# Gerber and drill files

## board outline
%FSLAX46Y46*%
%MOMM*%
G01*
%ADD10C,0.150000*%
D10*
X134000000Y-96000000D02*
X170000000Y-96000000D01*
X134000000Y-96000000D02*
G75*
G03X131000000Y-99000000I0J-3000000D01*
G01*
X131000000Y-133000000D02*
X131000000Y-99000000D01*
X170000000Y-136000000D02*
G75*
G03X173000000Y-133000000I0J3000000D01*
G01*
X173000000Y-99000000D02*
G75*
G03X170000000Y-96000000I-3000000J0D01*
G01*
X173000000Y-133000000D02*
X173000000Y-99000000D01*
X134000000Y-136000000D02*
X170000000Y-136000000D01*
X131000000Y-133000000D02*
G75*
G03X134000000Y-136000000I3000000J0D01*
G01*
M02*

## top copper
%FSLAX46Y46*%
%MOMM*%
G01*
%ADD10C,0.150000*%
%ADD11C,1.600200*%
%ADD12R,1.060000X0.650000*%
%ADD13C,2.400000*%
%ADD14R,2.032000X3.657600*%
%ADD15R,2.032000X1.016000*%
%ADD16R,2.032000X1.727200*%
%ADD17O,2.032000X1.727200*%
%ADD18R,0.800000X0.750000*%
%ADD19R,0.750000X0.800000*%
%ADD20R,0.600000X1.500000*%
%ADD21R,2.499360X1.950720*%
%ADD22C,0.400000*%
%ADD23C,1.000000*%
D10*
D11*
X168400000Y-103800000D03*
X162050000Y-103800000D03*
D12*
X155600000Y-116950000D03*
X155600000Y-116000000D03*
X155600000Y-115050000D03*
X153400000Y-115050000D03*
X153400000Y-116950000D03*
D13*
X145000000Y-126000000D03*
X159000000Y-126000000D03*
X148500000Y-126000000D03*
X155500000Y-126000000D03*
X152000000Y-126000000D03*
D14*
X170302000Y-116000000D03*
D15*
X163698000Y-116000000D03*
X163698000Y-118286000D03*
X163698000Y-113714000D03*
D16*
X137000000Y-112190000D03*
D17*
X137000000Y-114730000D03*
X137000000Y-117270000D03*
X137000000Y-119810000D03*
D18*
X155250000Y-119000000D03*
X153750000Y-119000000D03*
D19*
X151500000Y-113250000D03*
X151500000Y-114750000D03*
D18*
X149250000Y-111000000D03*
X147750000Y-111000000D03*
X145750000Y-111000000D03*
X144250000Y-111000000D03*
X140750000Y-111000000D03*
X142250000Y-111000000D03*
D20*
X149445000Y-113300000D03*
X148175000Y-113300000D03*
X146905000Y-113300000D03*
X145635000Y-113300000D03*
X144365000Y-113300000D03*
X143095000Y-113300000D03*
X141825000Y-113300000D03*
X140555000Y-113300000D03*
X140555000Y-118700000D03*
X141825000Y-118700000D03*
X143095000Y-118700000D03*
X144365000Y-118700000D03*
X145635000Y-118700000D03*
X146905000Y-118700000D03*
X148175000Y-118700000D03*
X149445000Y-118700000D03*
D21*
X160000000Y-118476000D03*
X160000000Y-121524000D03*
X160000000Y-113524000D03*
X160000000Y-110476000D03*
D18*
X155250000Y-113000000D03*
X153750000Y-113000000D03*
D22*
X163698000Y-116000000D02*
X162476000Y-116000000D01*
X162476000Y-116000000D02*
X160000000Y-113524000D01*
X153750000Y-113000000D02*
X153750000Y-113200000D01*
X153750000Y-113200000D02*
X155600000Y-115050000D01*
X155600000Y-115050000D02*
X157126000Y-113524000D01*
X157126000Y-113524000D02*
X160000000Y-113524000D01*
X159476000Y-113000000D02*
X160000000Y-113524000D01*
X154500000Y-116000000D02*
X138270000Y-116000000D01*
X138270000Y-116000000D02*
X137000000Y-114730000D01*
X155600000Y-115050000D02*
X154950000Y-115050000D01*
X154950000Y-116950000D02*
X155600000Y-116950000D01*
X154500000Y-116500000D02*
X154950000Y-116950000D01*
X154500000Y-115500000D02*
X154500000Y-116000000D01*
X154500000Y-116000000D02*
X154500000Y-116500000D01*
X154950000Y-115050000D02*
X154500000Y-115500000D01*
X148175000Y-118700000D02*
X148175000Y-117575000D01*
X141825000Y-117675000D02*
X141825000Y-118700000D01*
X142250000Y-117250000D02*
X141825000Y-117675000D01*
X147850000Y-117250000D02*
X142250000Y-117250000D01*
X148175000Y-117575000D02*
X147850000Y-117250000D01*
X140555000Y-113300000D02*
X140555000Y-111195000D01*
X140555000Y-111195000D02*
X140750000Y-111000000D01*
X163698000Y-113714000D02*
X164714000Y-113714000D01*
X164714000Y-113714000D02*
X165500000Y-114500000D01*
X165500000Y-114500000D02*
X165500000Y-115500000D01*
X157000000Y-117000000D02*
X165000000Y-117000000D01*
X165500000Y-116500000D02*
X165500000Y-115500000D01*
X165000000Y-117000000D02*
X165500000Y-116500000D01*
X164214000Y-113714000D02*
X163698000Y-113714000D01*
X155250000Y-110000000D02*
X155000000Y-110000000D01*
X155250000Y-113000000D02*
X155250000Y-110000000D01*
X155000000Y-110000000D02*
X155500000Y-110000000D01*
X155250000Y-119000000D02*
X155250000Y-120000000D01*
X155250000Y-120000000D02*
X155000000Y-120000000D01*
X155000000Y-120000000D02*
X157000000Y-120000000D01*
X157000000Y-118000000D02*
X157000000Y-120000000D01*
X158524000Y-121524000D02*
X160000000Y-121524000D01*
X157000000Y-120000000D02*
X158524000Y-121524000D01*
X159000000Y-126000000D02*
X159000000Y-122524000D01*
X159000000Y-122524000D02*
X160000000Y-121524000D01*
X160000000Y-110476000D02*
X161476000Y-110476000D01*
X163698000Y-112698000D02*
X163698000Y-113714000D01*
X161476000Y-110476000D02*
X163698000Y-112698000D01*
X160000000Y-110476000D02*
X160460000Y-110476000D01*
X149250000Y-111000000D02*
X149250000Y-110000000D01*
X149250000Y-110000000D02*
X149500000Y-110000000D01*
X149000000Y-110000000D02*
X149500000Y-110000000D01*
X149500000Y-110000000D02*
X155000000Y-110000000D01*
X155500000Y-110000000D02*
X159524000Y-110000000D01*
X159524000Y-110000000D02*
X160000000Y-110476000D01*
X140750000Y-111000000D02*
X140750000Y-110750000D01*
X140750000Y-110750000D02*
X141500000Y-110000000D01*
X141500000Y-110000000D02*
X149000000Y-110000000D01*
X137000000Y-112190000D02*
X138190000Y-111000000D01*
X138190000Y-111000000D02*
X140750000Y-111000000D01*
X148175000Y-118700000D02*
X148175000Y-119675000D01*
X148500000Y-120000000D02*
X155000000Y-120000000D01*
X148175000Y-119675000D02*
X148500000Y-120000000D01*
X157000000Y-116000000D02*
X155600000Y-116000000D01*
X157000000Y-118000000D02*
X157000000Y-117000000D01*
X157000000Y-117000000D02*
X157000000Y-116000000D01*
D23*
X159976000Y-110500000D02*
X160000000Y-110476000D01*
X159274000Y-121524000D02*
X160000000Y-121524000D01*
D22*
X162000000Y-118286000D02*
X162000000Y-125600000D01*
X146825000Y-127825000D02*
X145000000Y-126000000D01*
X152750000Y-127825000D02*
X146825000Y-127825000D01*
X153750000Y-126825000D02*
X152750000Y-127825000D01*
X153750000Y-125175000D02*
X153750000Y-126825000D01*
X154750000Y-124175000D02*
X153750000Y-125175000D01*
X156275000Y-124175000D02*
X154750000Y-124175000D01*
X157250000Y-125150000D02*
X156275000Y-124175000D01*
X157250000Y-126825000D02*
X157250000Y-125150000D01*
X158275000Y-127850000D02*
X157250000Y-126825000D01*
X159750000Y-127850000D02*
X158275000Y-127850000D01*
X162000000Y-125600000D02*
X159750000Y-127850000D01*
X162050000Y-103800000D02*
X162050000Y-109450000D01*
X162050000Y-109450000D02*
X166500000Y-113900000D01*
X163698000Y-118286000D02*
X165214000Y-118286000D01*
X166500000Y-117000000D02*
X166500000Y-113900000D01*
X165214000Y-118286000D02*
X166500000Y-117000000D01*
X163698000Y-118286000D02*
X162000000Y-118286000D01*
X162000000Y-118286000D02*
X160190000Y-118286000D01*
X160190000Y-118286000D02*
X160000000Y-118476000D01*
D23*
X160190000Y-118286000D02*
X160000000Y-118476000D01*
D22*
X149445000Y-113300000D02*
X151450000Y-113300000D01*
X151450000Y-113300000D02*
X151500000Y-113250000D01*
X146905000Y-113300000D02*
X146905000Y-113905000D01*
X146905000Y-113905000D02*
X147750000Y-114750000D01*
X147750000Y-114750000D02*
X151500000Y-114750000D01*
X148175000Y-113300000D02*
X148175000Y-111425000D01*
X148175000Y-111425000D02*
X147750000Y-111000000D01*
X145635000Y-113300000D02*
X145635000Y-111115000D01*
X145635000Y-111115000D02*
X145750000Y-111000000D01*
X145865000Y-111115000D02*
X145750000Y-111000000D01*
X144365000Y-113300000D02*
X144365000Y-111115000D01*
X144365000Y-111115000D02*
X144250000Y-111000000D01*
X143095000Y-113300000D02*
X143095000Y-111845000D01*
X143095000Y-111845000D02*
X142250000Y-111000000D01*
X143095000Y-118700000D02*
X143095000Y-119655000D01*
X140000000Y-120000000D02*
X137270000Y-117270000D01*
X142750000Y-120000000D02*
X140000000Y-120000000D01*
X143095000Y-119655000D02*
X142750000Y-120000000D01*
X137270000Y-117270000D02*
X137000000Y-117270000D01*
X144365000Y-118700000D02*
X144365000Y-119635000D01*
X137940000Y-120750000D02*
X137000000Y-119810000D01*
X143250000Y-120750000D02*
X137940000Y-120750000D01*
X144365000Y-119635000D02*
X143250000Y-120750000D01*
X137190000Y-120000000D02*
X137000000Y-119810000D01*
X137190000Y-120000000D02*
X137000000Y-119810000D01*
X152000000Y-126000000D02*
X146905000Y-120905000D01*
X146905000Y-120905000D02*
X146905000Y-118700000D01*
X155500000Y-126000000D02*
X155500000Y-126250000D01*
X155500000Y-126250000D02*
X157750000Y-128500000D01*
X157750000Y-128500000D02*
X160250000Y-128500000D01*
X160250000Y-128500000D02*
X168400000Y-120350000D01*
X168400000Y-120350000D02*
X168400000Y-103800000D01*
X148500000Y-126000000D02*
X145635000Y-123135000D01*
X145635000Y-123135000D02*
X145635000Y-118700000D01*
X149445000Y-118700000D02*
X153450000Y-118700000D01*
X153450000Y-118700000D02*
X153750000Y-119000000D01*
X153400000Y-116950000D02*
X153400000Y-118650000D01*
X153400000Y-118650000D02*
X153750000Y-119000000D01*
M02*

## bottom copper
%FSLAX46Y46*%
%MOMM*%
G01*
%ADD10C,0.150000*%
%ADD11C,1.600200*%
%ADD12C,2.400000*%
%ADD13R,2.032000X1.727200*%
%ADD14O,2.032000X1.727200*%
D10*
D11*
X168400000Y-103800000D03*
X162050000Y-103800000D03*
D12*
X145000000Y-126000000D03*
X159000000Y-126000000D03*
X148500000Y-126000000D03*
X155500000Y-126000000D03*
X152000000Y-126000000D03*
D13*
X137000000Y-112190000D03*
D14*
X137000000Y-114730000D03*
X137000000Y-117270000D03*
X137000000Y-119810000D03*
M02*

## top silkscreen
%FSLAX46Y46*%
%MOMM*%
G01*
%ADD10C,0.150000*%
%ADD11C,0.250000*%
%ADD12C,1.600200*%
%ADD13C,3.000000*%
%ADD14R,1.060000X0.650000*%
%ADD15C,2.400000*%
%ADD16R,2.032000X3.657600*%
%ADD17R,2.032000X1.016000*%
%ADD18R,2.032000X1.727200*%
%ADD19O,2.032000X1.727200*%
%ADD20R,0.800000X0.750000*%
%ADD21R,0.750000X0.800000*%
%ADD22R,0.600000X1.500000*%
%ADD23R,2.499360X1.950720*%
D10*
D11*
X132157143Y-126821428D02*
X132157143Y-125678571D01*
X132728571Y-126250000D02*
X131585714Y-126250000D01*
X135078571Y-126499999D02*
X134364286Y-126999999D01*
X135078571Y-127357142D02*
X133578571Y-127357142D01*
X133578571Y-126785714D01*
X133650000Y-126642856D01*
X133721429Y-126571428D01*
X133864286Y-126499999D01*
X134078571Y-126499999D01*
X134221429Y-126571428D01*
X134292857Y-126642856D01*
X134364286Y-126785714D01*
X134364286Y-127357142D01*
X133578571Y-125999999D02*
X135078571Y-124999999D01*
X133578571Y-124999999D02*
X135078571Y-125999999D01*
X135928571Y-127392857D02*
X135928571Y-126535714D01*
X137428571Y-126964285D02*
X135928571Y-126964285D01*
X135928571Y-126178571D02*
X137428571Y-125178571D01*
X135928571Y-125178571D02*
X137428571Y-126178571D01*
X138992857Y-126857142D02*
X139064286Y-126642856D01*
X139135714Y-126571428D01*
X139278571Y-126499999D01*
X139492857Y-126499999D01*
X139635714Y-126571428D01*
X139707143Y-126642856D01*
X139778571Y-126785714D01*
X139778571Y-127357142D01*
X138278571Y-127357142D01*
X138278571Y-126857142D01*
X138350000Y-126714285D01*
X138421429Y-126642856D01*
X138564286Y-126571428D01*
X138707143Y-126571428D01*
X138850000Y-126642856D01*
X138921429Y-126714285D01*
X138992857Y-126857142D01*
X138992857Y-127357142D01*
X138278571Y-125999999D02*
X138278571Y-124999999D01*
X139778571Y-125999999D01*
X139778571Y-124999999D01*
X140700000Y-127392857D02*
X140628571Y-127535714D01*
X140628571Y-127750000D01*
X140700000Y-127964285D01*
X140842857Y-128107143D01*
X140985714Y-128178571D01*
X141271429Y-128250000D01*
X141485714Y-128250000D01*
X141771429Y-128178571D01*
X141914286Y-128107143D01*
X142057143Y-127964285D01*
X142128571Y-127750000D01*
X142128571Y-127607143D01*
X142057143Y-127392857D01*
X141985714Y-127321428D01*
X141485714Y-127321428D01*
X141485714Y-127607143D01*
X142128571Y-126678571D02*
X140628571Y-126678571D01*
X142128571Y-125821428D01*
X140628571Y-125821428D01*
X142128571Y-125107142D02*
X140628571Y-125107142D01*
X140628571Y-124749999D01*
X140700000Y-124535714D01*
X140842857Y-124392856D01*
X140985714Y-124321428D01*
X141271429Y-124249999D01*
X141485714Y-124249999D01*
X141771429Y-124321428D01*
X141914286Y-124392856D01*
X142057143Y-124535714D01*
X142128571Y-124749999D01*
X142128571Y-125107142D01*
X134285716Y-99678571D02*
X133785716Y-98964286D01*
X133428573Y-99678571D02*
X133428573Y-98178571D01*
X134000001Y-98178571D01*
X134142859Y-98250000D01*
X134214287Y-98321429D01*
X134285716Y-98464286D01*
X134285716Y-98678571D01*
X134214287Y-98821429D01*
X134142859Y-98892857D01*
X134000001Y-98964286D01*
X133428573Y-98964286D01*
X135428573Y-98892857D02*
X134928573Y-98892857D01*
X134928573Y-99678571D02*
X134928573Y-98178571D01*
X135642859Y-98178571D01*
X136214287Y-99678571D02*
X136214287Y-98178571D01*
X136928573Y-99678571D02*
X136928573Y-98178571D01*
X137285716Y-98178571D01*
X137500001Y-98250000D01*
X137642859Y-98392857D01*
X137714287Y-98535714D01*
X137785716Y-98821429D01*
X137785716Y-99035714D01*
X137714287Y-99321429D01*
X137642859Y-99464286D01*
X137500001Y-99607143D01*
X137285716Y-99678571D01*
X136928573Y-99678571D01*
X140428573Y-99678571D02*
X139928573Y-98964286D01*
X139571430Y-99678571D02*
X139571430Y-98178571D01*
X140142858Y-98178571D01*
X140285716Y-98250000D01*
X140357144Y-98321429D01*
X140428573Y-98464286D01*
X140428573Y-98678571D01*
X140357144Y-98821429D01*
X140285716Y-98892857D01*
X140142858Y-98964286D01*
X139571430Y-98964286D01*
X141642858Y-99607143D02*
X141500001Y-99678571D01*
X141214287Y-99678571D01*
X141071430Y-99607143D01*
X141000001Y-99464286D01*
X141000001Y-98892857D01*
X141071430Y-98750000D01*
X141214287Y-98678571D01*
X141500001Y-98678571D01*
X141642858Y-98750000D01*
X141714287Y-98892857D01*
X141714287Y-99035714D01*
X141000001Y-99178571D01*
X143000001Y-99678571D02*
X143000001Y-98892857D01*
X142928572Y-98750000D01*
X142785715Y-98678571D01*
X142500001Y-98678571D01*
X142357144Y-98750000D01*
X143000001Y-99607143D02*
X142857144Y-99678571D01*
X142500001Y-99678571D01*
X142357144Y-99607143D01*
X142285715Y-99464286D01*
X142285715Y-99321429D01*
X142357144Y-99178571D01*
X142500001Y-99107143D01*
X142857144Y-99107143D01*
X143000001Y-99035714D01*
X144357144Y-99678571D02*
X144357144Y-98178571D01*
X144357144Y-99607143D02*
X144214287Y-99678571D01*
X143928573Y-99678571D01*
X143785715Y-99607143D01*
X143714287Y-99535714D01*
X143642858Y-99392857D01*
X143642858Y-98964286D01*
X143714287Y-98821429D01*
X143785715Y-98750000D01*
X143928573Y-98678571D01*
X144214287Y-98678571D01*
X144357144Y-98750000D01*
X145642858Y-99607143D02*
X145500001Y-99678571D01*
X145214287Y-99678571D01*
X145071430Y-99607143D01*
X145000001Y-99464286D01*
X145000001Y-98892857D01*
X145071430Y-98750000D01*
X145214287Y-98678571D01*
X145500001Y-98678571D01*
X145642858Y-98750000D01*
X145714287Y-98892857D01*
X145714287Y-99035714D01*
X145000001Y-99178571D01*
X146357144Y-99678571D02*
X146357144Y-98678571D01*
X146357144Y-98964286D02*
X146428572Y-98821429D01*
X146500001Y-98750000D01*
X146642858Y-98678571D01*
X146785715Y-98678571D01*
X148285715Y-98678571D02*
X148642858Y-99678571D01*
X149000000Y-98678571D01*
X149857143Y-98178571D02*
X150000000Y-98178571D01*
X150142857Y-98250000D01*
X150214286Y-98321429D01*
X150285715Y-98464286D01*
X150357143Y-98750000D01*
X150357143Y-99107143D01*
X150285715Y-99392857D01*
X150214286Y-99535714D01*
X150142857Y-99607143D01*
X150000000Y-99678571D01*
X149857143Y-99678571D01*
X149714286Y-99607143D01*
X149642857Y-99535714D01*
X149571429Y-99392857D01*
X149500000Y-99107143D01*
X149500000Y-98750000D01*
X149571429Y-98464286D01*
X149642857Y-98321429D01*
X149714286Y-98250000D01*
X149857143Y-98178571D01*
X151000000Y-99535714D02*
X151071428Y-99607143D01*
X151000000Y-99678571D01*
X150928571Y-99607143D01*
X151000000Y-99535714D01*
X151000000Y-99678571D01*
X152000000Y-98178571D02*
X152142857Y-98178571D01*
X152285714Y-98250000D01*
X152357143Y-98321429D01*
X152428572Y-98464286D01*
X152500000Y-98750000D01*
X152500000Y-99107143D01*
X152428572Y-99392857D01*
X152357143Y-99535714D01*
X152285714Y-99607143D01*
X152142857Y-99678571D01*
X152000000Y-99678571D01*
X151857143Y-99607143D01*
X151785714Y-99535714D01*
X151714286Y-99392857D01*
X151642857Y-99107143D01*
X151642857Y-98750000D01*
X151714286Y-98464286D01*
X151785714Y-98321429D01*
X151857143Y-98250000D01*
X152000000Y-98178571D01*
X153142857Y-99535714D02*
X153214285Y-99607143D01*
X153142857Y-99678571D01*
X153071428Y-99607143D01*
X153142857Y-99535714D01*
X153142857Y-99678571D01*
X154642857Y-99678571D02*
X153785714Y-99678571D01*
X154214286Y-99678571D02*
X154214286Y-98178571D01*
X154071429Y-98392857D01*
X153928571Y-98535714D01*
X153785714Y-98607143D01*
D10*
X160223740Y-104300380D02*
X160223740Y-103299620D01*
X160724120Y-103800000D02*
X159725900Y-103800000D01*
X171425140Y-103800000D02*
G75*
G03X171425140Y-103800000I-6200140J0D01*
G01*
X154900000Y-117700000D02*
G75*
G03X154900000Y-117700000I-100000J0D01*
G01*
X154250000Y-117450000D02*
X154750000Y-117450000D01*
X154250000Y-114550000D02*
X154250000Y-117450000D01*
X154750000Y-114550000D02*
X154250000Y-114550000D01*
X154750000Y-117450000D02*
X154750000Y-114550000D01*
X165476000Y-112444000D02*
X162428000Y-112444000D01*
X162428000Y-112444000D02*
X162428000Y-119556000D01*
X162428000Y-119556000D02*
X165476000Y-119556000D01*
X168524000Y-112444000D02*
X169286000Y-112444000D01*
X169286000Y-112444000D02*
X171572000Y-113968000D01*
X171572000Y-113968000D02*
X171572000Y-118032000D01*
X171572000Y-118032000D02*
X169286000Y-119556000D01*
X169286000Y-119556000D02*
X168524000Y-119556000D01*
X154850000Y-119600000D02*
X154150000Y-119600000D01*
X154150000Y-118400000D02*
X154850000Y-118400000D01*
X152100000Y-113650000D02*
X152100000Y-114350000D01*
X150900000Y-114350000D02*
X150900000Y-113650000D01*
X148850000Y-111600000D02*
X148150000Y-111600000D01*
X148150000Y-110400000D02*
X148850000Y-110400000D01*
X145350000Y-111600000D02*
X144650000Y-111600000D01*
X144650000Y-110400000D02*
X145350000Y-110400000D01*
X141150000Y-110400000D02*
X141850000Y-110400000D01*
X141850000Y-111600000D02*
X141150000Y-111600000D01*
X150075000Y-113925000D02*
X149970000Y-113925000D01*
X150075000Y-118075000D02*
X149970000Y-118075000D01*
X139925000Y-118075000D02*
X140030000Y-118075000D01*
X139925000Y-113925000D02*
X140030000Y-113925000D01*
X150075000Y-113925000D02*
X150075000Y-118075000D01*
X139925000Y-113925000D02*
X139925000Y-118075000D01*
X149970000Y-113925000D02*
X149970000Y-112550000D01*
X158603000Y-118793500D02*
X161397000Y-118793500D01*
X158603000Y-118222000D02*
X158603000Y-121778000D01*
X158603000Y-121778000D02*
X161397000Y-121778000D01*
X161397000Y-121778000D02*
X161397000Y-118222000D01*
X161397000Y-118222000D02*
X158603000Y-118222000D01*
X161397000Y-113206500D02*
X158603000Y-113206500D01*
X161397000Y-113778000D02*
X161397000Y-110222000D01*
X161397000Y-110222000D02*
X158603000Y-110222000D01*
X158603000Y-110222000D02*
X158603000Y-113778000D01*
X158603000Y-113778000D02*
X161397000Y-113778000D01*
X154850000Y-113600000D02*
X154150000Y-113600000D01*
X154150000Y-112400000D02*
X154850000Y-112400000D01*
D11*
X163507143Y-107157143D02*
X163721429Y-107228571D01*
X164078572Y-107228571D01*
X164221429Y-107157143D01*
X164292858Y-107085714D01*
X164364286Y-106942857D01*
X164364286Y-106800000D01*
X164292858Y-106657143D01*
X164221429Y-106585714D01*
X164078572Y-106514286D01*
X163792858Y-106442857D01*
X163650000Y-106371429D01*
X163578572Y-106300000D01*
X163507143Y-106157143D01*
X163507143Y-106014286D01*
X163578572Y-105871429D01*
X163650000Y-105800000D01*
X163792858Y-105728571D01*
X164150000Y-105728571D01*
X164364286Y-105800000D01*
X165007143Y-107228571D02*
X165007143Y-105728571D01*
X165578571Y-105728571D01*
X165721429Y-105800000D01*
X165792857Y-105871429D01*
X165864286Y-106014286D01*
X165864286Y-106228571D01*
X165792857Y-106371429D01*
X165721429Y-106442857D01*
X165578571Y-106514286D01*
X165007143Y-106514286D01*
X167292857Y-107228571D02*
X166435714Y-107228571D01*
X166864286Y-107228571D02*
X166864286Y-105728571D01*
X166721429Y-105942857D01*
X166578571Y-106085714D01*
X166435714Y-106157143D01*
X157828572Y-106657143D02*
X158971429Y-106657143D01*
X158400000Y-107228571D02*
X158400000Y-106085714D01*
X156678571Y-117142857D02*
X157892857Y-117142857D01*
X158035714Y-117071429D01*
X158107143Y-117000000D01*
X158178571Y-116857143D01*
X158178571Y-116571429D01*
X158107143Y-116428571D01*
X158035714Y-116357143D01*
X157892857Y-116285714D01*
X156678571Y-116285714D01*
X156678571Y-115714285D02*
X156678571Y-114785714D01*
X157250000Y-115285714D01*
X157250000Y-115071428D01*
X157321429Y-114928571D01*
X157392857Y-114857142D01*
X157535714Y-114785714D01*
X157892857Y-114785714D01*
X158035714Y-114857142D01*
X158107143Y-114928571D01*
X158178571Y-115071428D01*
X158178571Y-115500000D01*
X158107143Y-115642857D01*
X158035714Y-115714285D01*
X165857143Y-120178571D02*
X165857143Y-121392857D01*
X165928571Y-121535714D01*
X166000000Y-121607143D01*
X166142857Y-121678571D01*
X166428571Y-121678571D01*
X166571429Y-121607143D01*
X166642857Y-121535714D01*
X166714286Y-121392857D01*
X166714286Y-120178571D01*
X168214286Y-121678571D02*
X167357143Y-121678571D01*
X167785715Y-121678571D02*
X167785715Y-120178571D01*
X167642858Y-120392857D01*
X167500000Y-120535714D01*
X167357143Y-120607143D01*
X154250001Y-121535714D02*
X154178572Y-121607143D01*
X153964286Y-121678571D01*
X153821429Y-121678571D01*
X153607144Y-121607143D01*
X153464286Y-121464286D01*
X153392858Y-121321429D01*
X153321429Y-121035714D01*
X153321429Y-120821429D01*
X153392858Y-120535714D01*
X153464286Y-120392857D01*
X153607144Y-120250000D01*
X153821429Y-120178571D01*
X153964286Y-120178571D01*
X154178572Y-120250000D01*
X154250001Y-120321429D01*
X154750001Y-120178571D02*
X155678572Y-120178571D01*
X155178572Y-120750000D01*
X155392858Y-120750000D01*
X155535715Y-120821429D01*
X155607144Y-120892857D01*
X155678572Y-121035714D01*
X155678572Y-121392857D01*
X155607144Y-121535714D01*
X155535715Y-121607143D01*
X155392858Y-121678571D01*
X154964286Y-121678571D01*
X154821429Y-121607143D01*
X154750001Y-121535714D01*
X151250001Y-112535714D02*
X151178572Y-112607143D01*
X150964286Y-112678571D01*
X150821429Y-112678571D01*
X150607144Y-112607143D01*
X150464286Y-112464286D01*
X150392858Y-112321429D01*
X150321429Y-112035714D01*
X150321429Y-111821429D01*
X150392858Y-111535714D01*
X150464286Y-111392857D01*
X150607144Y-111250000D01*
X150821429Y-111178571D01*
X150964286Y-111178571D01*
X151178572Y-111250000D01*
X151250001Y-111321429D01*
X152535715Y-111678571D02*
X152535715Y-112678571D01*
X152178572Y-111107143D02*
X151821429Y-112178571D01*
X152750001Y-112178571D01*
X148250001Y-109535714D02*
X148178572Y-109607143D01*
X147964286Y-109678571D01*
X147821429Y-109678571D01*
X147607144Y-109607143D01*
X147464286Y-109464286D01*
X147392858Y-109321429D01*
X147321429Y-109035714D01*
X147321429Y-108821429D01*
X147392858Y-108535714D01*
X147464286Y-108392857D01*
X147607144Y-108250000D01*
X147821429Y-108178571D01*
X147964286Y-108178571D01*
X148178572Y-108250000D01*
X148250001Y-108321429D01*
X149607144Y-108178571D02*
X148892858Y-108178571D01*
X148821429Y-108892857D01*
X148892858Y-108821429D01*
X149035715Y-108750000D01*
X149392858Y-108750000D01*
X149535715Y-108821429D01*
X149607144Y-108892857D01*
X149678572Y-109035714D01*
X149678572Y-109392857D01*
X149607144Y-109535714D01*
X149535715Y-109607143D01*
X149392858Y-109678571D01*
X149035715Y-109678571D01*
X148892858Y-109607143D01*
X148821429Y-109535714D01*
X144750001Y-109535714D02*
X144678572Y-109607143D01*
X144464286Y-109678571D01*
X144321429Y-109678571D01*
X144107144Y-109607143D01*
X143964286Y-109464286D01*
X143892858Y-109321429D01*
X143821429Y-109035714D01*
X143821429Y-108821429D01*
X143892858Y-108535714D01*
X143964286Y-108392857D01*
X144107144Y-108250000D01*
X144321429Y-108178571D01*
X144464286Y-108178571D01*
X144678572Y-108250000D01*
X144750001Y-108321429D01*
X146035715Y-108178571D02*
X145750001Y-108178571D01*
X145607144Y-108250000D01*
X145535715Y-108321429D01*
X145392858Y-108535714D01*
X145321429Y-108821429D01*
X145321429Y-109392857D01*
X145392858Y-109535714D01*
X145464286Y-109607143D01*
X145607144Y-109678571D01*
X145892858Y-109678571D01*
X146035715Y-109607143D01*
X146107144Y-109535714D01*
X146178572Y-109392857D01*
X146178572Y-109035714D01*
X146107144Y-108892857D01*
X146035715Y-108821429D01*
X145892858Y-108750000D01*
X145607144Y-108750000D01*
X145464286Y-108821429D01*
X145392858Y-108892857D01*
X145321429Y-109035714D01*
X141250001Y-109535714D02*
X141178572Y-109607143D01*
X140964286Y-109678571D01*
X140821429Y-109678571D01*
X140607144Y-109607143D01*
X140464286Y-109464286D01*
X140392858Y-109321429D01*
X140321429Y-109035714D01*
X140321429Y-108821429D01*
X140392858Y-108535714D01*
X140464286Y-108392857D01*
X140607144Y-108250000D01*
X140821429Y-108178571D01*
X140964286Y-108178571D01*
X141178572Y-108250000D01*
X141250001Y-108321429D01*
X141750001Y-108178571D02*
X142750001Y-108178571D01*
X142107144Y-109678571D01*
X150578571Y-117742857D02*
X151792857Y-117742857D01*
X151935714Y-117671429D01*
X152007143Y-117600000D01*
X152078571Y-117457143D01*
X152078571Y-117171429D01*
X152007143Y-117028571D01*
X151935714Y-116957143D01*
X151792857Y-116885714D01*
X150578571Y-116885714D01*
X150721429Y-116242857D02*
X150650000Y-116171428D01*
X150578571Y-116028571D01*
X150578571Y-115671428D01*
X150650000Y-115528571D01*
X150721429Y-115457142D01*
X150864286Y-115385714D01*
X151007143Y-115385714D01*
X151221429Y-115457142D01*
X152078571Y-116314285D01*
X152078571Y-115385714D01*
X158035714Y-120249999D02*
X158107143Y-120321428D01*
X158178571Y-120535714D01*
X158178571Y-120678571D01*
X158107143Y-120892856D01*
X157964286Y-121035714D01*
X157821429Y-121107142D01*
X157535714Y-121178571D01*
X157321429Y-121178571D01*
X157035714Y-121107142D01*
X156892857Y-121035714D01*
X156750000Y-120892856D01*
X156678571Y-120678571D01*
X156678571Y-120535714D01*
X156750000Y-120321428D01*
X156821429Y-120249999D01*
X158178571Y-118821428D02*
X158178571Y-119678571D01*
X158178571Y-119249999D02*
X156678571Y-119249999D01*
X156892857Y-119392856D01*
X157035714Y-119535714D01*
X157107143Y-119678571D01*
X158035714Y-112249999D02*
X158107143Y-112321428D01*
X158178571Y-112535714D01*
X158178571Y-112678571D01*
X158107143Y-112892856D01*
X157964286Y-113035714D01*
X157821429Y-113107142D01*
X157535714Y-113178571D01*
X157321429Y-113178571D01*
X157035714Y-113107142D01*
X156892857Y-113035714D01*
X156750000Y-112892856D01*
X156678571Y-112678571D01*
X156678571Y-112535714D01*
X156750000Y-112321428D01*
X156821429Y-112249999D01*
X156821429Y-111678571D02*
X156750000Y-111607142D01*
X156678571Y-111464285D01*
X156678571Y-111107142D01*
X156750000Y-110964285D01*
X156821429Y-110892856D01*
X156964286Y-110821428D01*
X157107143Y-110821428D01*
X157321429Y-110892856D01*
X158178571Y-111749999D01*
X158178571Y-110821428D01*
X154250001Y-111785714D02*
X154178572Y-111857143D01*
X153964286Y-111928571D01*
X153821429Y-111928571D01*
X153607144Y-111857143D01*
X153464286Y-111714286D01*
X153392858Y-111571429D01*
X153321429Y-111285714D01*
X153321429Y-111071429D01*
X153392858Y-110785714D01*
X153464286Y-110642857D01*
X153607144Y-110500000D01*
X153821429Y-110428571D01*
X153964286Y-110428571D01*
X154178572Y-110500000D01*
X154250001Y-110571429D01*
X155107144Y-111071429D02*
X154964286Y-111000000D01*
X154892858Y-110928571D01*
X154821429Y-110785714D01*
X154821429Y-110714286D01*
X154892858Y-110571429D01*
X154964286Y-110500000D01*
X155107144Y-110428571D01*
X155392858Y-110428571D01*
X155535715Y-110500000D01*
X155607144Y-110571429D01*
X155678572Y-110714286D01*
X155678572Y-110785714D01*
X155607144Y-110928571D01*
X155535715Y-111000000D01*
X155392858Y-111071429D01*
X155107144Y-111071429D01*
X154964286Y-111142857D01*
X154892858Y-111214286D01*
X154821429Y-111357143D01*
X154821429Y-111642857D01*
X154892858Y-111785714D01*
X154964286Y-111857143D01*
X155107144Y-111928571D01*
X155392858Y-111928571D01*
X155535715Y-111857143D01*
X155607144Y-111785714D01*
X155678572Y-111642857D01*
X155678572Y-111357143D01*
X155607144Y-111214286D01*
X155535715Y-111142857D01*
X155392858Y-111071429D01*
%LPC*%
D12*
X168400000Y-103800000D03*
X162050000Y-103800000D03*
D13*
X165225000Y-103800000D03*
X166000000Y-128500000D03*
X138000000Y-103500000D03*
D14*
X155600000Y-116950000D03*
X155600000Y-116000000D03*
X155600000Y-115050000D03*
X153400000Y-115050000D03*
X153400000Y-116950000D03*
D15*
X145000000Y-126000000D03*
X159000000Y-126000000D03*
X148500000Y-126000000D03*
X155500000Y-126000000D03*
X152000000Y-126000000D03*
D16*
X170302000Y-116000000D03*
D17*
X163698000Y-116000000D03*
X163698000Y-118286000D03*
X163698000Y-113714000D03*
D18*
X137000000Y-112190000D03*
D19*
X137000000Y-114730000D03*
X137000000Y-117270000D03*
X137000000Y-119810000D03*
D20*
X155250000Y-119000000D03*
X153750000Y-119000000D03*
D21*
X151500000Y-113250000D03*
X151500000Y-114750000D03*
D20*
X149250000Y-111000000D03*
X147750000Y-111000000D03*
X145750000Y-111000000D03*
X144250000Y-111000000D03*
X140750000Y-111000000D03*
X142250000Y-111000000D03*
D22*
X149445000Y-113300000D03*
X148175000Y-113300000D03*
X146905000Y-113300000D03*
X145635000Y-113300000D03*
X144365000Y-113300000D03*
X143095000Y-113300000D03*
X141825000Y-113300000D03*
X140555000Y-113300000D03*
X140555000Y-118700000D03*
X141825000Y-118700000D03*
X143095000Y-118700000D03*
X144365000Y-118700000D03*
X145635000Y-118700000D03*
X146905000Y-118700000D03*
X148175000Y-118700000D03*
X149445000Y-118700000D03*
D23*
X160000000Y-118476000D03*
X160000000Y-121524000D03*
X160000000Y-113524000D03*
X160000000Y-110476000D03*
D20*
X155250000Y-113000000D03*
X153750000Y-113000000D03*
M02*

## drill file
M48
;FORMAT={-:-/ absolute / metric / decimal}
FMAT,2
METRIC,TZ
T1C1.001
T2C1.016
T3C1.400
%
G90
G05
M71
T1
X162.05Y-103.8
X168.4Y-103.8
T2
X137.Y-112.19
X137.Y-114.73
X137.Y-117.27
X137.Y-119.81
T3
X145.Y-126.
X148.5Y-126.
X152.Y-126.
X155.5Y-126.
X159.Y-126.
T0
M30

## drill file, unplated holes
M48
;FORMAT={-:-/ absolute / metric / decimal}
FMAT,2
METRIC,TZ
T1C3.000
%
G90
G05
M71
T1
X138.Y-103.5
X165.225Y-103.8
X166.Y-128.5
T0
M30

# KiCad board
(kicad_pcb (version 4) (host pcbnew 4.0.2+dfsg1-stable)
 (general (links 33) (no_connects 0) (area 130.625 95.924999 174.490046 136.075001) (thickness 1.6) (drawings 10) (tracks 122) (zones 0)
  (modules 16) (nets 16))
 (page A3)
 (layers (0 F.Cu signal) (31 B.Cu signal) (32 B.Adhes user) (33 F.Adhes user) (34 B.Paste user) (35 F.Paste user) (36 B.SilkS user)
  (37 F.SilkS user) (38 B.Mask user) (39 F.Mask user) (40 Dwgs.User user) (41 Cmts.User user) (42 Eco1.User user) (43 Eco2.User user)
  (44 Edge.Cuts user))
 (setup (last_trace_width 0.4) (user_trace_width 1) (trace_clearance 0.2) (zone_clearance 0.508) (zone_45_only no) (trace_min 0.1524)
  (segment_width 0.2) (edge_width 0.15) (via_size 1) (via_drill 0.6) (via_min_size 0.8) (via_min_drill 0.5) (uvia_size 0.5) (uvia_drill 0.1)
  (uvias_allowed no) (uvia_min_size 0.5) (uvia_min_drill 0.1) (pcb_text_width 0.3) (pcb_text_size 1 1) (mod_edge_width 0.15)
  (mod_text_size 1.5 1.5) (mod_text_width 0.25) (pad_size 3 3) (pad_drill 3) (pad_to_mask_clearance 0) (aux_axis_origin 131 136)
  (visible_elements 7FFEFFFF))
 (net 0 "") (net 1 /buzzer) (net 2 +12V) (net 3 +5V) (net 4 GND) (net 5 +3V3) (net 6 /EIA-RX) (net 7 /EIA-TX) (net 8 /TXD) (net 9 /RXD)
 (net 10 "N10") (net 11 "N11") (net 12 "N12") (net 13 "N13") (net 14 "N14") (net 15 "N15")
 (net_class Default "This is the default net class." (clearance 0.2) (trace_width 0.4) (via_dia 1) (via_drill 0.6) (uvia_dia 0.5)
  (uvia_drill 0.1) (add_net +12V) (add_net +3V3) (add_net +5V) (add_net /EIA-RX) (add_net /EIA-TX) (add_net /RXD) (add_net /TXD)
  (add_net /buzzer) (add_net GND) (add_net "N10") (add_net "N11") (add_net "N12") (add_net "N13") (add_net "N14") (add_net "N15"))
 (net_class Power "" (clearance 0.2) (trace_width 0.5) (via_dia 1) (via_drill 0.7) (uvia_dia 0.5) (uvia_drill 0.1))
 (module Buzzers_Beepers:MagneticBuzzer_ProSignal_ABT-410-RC (layer F.Cu) (at 168.4 103.8 180)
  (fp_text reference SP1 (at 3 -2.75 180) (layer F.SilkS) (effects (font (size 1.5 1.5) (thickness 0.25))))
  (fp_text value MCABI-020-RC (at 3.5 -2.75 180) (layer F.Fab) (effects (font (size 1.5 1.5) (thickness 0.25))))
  (fp_line (start 8.17626 -0.50038) (end 8.17626 0.50038) (layer F.SilkS) (width 0.15))
  (fp_line (start 7.67588 0) (end 8.6741 0) (layer F.SilkS) (width 0.15))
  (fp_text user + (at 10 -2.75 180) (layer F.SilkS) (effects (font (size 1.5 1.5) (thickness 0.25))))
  (fp_circle (center 3.175 0) (end 9.37514 0) (layer F.SilkS) (width 0.15))
  (pad 1 thru_hole circle (at 0 0 180) (size 1.6002 1.6002) (drill 1.00076) (layers *.Cu *.Mask F.SilkS) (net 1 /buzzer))
  (pad 2 thru_hole circle (at 6.35 0 180) (size 1.6002 1.6002) (drill 1.00076) (layers *.Cu *.Mask F.SilkS) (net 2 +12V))
  (pad "" np_thru_hole circle (at 3.175 0 180) (size 3 3) (drill 3) (layers *.Cu *.Mask)))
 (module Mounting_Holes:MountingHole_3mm (layer F.Cu) (at 166 128.5)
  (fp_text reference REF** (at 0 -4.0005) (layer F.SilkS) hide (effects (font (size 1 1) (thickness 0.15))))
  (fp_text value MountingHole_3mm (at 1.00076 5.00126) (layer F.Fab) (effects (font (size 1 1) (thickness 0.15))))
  (pad "" np_thru_hole circle (at 0 0) (size 3 3) (drill 3) (layers *.Cu *.Mask)))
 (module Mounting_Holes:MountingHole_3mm (layer F.Cu) (at 138 103.5)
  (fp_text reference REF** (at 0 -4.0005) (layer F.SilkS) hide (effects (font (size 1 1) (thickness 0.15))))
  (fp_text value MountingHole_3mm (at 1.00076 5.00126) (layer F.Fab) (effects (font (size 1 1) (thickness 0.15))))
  (pad "" np_thru_hole circle (at 0 0) (size 3 3) (drill 3) (layers *.Cu *.Mask)))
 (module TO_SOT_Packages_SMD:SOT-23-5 (layer F.Cu) (at 154.5 116 180)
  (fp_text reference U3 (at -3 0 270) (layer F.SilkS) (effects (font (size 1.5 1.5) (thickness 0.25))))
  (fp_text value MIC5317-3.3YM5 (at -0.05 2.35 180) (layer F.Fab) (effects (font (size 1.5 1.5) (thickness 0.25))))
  (fp_circle (center -0.3 -1.7) (end -0.2 -1.7) (layer F.SilkS) (width 0.15))
  (fp_line (start 0.25 -1.45) (end -0.25 -1.45) (layer F.SilkS) (width 0.15))
  (fp_line (start 0.25 1.45) (end 0.25 -1.45) (layer F.SilkS) (width 0.15))
  (fp_line (start -0.25 1.45) (end 0.25 1.45) (layer F.SilkS) (width 0.15))
  (fp_line (start -0.25 -1.45) (end -0.25 1.45) (layer F.SilkS) (width 0.15))
  (pad VI smd rect (at -1.1 -0.95 180) (size 1.06 0.65) (layers F.Cu F.Paste F.Mask) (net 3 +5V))
  (pad GND smd rect (at -1.1 0 180) (size 1.06 0.65) (layers F.Cu F.Paste F.Mask) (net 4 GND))
  (pad VI smd rect (at -1.1 0.95 180) (size 1.06 0.65) (layers F.Cu F.Paste F.Mask) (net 3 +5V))
  (pad NC smd rect (at 1.1 0.95 180) (size 1.06 0.65) (layers F.Cu F.Paste F.Mask))
  (pad VO smd rect (at 1.1 -0.95 180) (size 1.06 0.65) (layers F.Cu F.Paste F.Mask) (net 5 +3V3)))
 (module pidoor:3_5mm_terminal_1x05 (layer F.Cu) (at 152 126 270)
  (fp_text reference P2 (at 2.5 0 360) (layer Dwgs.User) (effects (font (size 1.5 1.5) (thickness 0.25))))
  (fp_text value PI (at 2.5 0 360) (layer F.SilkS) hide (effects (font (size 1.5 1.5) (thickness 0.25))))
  (pad 5 thru_hole circle (at 0 7 270) (size 2.4 2.4) (drill 1.4) (layers *.Cu *.Mask) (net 2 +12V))
  (pad 1 thru_hole circle (at 0 -7 270) (size 2.4 2.4) (drill 1.4) (layers *.Cu *.Mask) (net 4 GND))
  (pad 4 thru_hole circle (at 0 3.5 270) (size 2.4 2.4) (drill 1.4) (layers *.Cu *.Mask) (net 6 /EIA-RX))
  (pad 2 thru_hole circle (at 0 -3.5 270) (size 2.4 2.4) (drill 1.4) (layers *.Cu *.Mask) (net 1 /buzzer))
  (pad 3 thru_hole circle (at 0 0 270) (size 2.4 2.4) (drill 1.4) (layers *.Cu *.Mask) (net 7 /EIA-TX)))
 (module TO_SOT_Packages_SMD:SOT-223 (layer F.Cu) (at 167 116 270)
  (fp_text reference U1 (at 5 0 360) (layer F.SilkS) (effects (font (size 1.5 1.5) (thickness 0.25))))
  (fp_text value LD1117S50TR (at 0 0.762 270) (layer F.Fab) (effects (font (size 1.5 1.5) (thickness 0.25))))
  (fp_line (start -3.556 1.524) (end -3.556 4.572) (layer F.SilkS) (width 0.15))
  (fp_line (start -3.556 4.572) (end 3.556 4.572) (layer F.SilkS) (width 0.15))
  (fp_line (start 3.556 4.572) (end 3.556 1.524) (layer F.SilkS) (width 0.15))
  (fp_line (start -3.556 -1.524) (end -3.556 -2.286) (layer F.SilkS) (width 0.15))
  (fp_line (start -3.556 -2.286) (end -2.032 -4.572) (layer F.SilkS) (width 0.15))
  (fp_line (start -2.032 -4.572) (end 2.032 -4.572) (layer F.SilkS) (width 0.15))
  (fp_line (start 2.032 -4.572) (end 3.556 -2.286) (layer F.SilkS) (width 0.15))
  (fp_line (start 3.556 -2.286) (end 3.556 -1.524) (layer F.SilkS) (width 0.15))
  (pad NC smd rect (at 0 -3.302 270) (size 3.6576 2.032) (layers F.Cu F.Paste F.Mask))
  (pad VO smd rect (at 0 3.302 270) (size 1.016 2.032) (layers F.Cu F.Paste F.Mask) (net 3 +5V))
  (pad VI smd rect (at 2.286 3.302 270) (size 1.016 2.032) (layers F.Cu F.Paste F.Mask) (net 2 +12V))
  (pad GND smd rect (at -2.286 3.302 270) (size 1.016 2.032) (layers F.Cu F.Paste F.Mask) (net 4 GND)))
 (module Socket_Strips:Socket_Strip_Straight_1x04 (layer B.Cu) (at 137 116 270)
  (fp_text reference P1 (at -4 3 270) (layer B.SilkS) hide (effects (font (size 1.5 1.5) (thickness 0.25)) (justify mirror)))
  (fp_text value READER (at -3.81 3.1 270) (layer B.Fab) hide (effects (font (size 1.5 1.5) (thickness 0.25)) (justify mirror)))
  (pad 1 thru_hole rect (at -3.81 0 270) (size 1.7272 2.032) (drill 1.016) (layers *.Cu *.Mask) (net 4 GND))
  (pad 2 thru_hole oval (at -1.27 0 270) (size 1.7272 2.032) (drill 1.016) (layers *.Cu *.Mask) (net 3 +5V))
  (pad 3 thru_hole oval (at 1.27 0 270) (size 1.7272 2.032) (drill 1.016) (layers *.Cu *.Mask) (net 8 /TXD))
  (pad 4 thru_hole oval (at 3.81 0 270) (size 1.7272 2.032) (drill 1.016) (layers *.Cu *.Mask) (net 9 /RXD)))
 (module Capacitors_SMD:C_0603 (layer F.Cu) (at 154.5 119 180)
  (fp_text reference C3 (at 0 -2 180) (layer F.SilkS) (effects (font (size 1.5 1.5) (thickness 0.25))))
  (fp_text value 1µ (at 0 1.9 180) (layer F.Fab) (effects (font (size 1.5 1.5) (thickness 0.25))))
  (fp_line (start -0.35 -0.6) (end 0.35 -0.6) (layer F.SilkS) (width 0.15))
  (fp_line (start 0.35 0.6) (end -0.35 0.6) (layer F.SilkS) (width 0.15))
  (pad 1 smd rect (at -0.75 0 180) (size 0.8 0.75) (layers F.Cu F.Paste F.Mask) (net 4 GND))
  (pad 2 smd rect (at 0.75 0 180) (size 0.8 0.75) (layers F.Cu F.Paste F.Mask) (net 5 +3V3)))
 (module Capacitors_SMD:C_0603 (layer F.Cu) (at 151.5 114 270)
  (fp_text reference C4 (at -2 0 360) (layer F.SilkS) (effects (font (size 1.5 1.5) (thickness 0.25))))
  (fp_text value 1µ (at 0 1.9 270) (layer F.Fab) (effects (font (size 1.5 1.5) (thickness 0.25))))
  (fp_line (start -0.35 -0.6) (end 0.35 -0.6) (layer F.SilkS) (width 0.15))
  (fp_line (start 0.35 0.6) (end -0.35 0.6) (layer F.SilkS) (width 0.15))
  (pad 1 smd rect (at -0.75 0 270) (size 0.8 0.75) (layers F.Cu F.Paste F.Mask) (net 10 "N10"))
  (pad 2 smd rect (at 0.75 0 270) (size 0.8 0.75) (layers F.Cu F.Paste F.Mask) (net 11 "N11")))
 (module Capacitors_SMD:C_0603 (layer F.Cu) (at 148.5 111 180)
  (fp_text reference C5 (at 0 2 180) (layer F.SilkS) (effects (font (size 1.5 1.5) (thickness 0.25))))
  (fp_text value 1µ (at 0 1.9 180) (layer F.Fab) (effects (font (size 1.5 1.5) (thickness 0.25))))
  (fp_line (start -0.35 -0.6) (end 0.35 -0.6) (layer F.SilkS) (width 0.15))
  (fp_line (start 0.35 0.6) (end -0.35 0.6) (layer F.SilkS) (width 0.15))
  (pad 1 smd rect (at -0.75 0 180) (size 0.8 0.75) (layers F.Cu F.Paste F.Mask) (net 4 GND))
  (pad 2 smd rect (at 0.75 0 180) (size 0.8 0.75) (layers F.Cu F.Paste F.Mask) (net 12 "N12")))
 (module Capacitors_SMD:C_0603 (layer F.Cu) (at 145 111 180)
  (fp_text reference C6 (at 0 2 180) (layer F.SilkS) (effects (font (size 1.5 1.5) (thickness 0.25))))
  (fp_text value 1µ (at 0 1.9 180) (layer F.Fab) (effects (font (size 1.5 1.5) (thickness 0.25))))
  (fp_line (start -0.35 -0.6) (end 0.35 -0.6) (layer F.SilkS) (width 0.15))
  (fp_line (start 0.35 0.6) (end -0.35 0.6) (layer F.SilkS) (width 0.15))
  (pad 1 smd rect (at -0.75 0 180) (size 0.8 0.75) (layers F.Cu F.Paste F.Mask) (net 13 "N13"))
  (pad 2 smd rect (at 0.75 0 180) (size 0.8 0.75) (layers F.Cu F.Paste F.Mask) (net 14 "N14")))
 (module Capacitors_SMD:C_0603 (layer F.Cu) (at 141.5 111)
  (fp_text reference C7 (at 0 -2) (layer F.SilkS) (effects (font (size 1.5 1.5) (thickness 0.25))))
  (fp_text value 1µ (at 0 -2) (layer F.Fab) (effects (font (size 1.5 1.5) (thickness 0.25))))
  (fp_line (start -0.35 -0.6) (end 0.35 -0.6) (layer F.SilkS) (width 0.15))
  (fp_line (start 0.35 0.6) (end -0.35 0.6) (layer F.SilkS) (width 0.15))
  (pad 1 smd rect (at -0.75 0) (size 0.8 0.75) (layers F.Cu F.Paste F.Mask) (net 4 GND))
  (pad 2 smd rect (at 0.75 0) (size 0.8 0.75) (layers F.Cu F.Paste F.Mask) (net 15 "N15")))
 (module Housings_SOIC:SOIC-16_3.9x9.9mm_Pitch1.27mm (layer F.Cu) (at 145 116 270)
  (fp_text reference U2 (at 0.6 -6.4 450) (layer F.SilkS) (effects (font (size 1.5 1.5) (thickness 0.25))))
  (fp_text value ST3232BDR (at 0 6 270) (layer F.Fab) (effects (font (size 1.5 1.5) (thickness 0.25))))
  (fp_line (start -2.075 -5.075) (end -2.075 -4.97) (layer F.SilkS) (width 0.15))
  (fp_line (start 2.075 -5.075) (end 2.075 -4.97) (layer F.SilkS) (width 0.15))
  (fp_line (start 2.075 5.075) (end 2.075 4.97) (layer F.SilkS) (width 0.15))
  (fp_line (start -2.075 5.075) (end -2.075 4.97) (layer F.SilkS) (width 0.15))
  (fp_line (start -2.075 -5.075) (end 2.075 -5.075) (layer F.SilkS) (width 0.15))
  (fp_line (start -2.075 5.075) (end 2.075 5.075) (layer F.SilkS) (width 0.15))
  (fp_line (start -2.075 -4.97) (end -3.45 -4.97) (layer F.SilkS) (width 0.15))
  (pad 1 smd rect (at -2.7 -4.445 270) (size 1.5 0.6) (layers F.Cu F.Paste F.Mask) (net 10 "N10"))
  (pad 2 smd rect (at -2.7 -3.175 270) (size 1.5 0.6) (layers F.Cu F.Paste F.Mask) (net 12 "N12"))
  (pad 3 smd rect (at -2.7 -1.905 270) (size 1.5 0.6) (layers F.Cu F.Paste F.Mask) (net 11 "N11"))
  (pad 4 smd rect (at -2.7 -0.635 270) (size 1.5 0.6) (layers F.Cu F.Paste F.Mask) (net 13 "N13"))
  (pad 5 smd rect (at -2.7 0.635 270) (size 1.5 0.6) (layers F.Cu F.Paste F.Mask) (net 14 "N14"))
  (pad 6 smd rect (at -2.7 1.905 270) (size 1.5 0.6) (layers F.Cu F.Paste F.Mask) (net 15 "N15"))
  (pad 7 smd rect (at -2.7 3.175 270) (size 1.5 0.6) (layers F.Cu F.Paste F.Mask))
  (pad 8 smd rect (at -2.7 4.445 270) (size 1.5 0.6) (layers F.Cu F.Paste F.Mask) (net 4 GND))
  (pad 9 smd rect (at 2.7 4.445 270) (size 1.5 0.6) (layers F.Cu F.Paste F.Mask))
  (pad 10 smd rect (at 2.7 3.175 270) (size 1.5 0.6) (layers F.Cu F.Paste F.Mask) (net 4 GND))
  (pad 11 smd rect (at 2.7 1.905 270) (size 1.5 0.6) (layers F.Cu F.Paste F.Mask) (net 8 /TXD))
  (pad 12 smd rect (at 2.7 0.635 270) (size 1.5 0.6) (layers F.Cu F.Paste F.Mask) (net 9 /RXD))
  (pad 13 smd rect (at 2.7 -0.635 270) (size 1.5 0.6) (layers F.Cu F.Paste F.Mask) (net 6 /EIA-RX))
  (pad 14 smd rect (at 2.7 -1.905 270) (size 1.5 0.6) (layers F.Cu F.Paste F.Mask) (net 7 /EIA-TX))
  (pad 15 smd rect (at 2.7 -3.175 270) (size 1.5 0.6) (layers F.Cu F.Paste F.Mask) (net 4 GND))
  (pad 16 smd rect (at 2.7 -4.445 270) (size 1.5 0.6) (layers F.Cu F.Paste F.Mask) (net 5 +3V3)))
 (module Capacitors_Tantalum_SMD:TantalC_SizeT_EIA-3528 (layer F.Cu) (at 160 120 90)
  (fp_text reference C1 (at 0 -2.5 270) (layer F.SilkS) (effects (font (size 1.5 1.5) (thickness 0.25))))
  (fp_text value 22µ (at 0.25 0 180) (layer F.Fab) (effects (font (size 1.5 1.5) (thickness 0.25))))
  (fp_line (start 1.2065 -1.397) (end 1.2065 1.397) (layer F.SilkS) (width 0.15))
  (fp_line (start 1.778 -1.397) (end -1.778 -1.397) (layer F.SilkS) (width 0.15))
  (fp_line (start -1.778 -1.397) (end -1.778 1.397) (layer F.SilkS) (width 0.15))
  (fp_line (start -1.778 1.397) (end 1.778 1.397) (layer F.SilkS) (width 0.15))
  (fp_line (start 1.778 1.397) (end 1.778 -1.397) (layer F.SilkS) (width 0.15))
  (pad 1 smd rect (at 1.524 0 90) (size 1.95072 2.49936) (layers F.Cu F.Paste F.Mask) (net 2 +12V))
  (pad 2 smd rect (at -1.524 0 90) (size 1.95072 2.49936) (layers F.Cu F.Paste F.Mask) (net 4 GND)))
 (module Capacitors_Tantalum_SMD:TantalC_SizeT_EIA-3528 (layer F.Cu) (at 160 112 270)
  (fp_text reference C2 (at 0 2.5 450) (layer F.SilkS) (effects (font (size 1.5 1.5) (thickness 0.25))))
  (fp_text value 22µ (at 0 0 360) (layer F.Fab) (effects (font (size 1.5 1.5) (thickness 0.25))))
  (fp_line (start 1.2065 -1.397) (end 1.2065 1.397) (layer F.SilkS) (width 0.15))
  (fp_line (start 1.778 -1.397) (end -1.778 -1.397) (layer F.SilkS) (width 0.15))
  (fp_line (start -1.778 -1.397) (end -1.778 1.397) (layer F.SilkS) (width 0.15))
  (fp_line (start -1.778 1.397) (end 1.778 1.397) (layer F.SilkS) (width 0.15))
  (fp_line (start 1.778 1.397) (end 1.778 -1.397) (layer F.SilkS) (width 0.15))
  (pad 1 smd rect (at 1.524 0 270) (size 1.95072 2.49936) (layers F.Cu F.Paste F.Mask) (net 3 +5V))
  (pad 2 smd rect (at -1.524 0 270) (size 1.95072 2.49936) (layers F.Cu F.Paste F.Mask) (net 4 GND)))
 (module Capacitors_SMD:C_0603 (layer F.Cu) (at 154.5 113 180)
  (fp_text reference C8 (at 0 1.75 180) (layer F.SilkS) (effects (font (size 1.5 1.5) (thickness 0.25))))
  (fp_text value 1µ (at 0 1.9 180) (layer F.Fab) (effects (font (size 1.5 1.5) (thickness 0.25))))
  (fp_line (start -0.35 -0.6) (end 0.35 -0.6) (layer F.SilkS) (width 0.15))
  (fp_line (start 0.35 0.6) (end -0.35 0.6) (layer F.SilkS) (width 0.15))
  (pad 1 smd rect (at -0.75 0 180) (size 0.8 0.75) (layers F.Cu F.Paste F.Mask) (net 4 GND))
  (pad 2 smd rect (at 0.75 0 180) (size 0.8 0.75) (layers F.Cu F.Paste F.Mask) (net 3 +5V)))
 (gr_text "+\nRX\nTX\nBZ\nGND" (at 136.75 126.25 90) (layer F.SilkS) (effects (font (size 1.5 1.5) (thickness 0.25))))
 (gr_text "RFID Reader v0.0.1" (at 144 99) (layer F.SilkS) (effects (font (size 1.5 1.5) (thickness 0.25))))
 (gr_line (start 134 96) (end 170 96) (angle 90) (layer Edge.Cuts) (width 0.15))
 (gr_arc (start 134 99) (end 131 99) (angle 90) (layer Edge.Cuts) (width 0.15))
 (gr_line (start 131 133) (end 131 99) (angle 90) (layer Edge.Cuts) (width 0.15))
 (gr_arc (start 170 133) (end 173 133) (angle 90) (layer Edge.Cuts) (width 0.15))
 (gr_arc (start 170 99) (end 170 96) (angle 90) (layer Edge.Cuts) (width 0.15))
 (gr_line (start 173 133) (end 173 99) (angle 90) (layer Edge.Cuts) (width 0.15))
 (gr_line (start 134 136) (end 170 136) (angle 90) (layer Edge.Cuts) (width 0.15))
 (gr_arc (start 134 133) (end 134 136) (angle 90) (layer Edge.Cuts) (width 0.15))
 (segment (start 163.698 116) (end 162.476 116) (width 0.4) (layer F.Cu) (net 3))
 (segment (start 162.476 116) (end 160 113.524) (width 0.4) (layer F.Cu) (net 3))
 (segment (start 153.75 113) (end 153.75 113.2) (width 0.4) (layer F.Cu) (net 3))
 (segment (start 153.75 113.2) (end 155.6 115.05) (width 0.4) (layer F.Cu) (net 3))
 (segment (start 155.6 115.05) (end 157.126 113.524) (width 0.4) (layer F.Cu) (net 3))
 (segment (start 157.126 113.524) (end 160 113.524) (width 0.4) (layer F.Cu) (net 3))
 (segment (start 159.476 113) (end 160 113.524) (width 0.4) (layer F.Cu) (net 3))
 (segment (start 154.5 116) (end 138.27 116) (width 0.4) (layer F.Cu) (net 3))
 (segment (start 138.27 116) (end 137 114.73) (width 0.4) (layer F.Cu) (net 3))
 (segment (start 155.6 115.05) (end 154.95 115.05) (width 0.4) (layer F.Cu) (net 3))
 (segment (start 154.95 116.95) (end 155.6 116.95) (width 0.4) (layer F.Cu) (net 3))
 (segment (start 154.5 116.5) (end 154.95 116.95) (width 0.4) (layer F.Cu) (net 3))
 (segment (start 154.5 115.5) (end 154.5 116) (width 0.4) (layer F.Cu) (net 3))
 (segment (start 154.5 116) (end 154.5 116.5) (width 0.4) (layer F.Cu) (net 3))
 (segment (start 154.95 115.05) (end 154.5 115.5) (width 0.4) (layer F.Cu) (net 3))
 (segment (start 148.175 118.7) (end 148.175 117.575) (width 0.4) (layer F.Cu) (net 4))
 (segment (start 141.825 117.675) (end 141.825 118.7) (width 0.4) (layer F.Cu) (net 4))
 (segment (start 142.25 117.25) (end 141.825 117.675) (width 0.4) (layer F.Cu) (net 4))
 (segment (start 147.85 117.25) (end 142.25 117.25) (width 0.4) (layer F.Cu) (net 4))
 (segment (start 148.175 117.575) (end 147.85 117.25) (width 0.4) (layer F.Cu) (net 4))
 (segment (start 140.555 113.3) (end 140.555 111.195) (width 0.4) (layer F.Cu) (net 4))
 (segment (start 140.555 111.195) (end 140.75 111) (width 0.4) (layer F.Cu) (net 4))
 (segment (start 163.698 113.714) (end 164.714 113.714) (width 0.4) (layer F.Cu) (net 4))
 (segment (start 164.714 113.714) (end 165.5 114.5) (width 0.4) (layer F.Cu) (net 4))
 (segment (start 165.5 114.5) (end 165.5 115.5) (width 0.4) (layer F.Cu) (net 4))
 (segment (start 157 117) (end 165 117) (width 0.4) (layer F.Cu) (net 4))
 (segment (start 165.5 116.5) (end 165.5 115.5) (width 0.4) (layer F.Cu) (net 4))
 (segment (start 165 117) (end 165.5 116.5) (width 0.4) (layer F.Cu) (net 4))
 (segment (start 164.214 113.714) (end 163.698 113.714) (width 0.4) (layer F.Cu) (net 4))
 (segment (start 155.25 110) (end 155 110) (width 0.4) (layer F.Cu) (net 4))
 (segment (start 155.25 113) (end 155.25 110) (width 0.4) (layer F.Cu) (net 4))
 (segment (start 155 110) (end 155.5 110) (width 0.4) (layer F.Cu) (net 4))
 (segment (start 155.25 119) (end 155.25 120) (width 0.4) (layer F.Cu) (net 4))
 (segment (start 155.25 120) (end 155 120) (width 0.4) (layer F.Cu) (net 4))
 (segment (start 155 120) (end 157 120) (width 0.4) (layer F.Cu) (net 4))
 (segment (start 157 118) (end 157 120) (width 0.4) (layer F.Cu) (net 4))
 (segment (start 158.524 121.524) (end 160 121.524) (width 0.4) (layer F.Cu) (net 4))
 (segment (start 157 120) (end 158.524 121.524) (width 0.4) (layer F.Cu) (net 4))
 (segment (start 159 126) (end 159 122.524) (width 0.4) (layer F.Cu) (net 4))
 (segment (start 159 122.524) (end 160 121.524) (width 0.4) (layer F.Cu) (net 4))
 (segment (start 160 110.476) (end 161.476 110.476) (width 0.4) (layer F.Cu) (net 4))
 (segment (start 163.698 112.698) (end 163.698 113.714) (width 0.4) (layer F.Cu) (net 4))
 (segment (start 161.476 110.476) (end 163.698 112.698) (width 0.4) (layer F.Cu) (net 4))
 (segment (start 160 110.476) (end 160.46 110.476) (width 0.4) (layer F.Cu) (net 4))
 (segment (start 149.25 111) (end 149.25 110) (width 0.4) (layer F.Cu) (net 4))
 (segment (start 149.25 110) (end 149.5 110) (width 0.4) (layer F.Cu) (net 4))
 (segment (start 149 110) (end 149.5 110) (width 0.4) (layer F.Cu) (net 4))
 (segment (start 149.5 110) (end 155 110) (width 0.4) (layer F.Cu) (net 4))
 (segment (start 155.5 110) (end 159.524 110) (width 0.4) (layer F.Cu) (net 4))
 (segment (start 159.524 110) (end 160 110.476) (width 0.4) (layer F.Cu) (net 4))
 (segment (start 140.75 111) (end 140.75 110.75) (width 0.4) (layer F.Cu) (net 4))
 (segment (start 140.75 110.75) (end 141.5 110) (width 0.4) (layer F.Cu) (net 4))
 (segment (start 141.5 110) (end 149 110) (width 0.4) (layer F.Cu) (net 4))
 (segment (start 137 112.19) (end 138.19 111) (width 0.4) (layer F.Cu) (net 4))
 (segment (start 138.19 111) (end 140.75 111) (width 0.4) (layer F.Cu) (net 4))
 (segment (start 148.175 118.7) (end 148.175 119.675) (width 0.4) (layer F.Cu) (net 4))
 (segment (start 148.5 120) (end 155 120) (width 0.4) (layer F.Cu) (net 4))
 (segment (start 148.175 119.675) (end 148.5 120) (width 0.4) (layer F.Cu) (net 4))
 (segment (start 157 116) (end 155.6 116) (width 0.4) (layer F.Cu) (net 4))
 (segment (start 157 118) (end 157 117) (width 0.4) (layer F.Cu) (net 4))
 (segment (start 157 117) (end 157 116) (width 0.4) (layer F.Cu) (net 4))
 (segment (start 159.976 110.5) (end 160 110.476) (width 1) (layer F.Cu) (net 4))
 (segment (start 159.274 121.524) (end 160 121.524) (width 1) (layer F.Cu) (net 4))
 (segment (start 162 118.286) (end 162 125.6) (width 0.4) (layer F.Cu) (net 2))
 (segment (start 146.825 127.825) (end 145 126) (width 0.4) (layer F.Cu) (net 2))
 (segment (start 152.75 127.825) (end 146.825 127.825) (width 0.4) (layer F.Cu) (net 2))
 (segment (start 153.75 126.825) (end 152.75 127.825) (width 0.4) (layer F.Cu) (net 2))
 (segment (start 153.75 125.175) (end 153.75 126.825) (width 0.4) (layer F.Cu) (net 2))
 (segment (start 154.75 124.175) (end 153.75 125.175) (width 0.4) (layer F.Cu) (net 2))
 (segment (start 156.275 124.175) (end 154.75 124.175) (width 0.4) (layer F.Cu) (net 2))
 (segment (start 157.25 125.15) (end 156.275 124.175) (width 0.4) (layer F.Cu) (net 2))
 (segment (start 157.25 126.825) (end 157.25 125.15) (width 0.4) (layer F.Cu) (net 2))
 (segment (start 158.275 127.85) (end 157.25 126.825) (width 0.4) (layer F.Cu) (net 2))
 (segment (start 159.75 127.85) (end 158.275 127.85) (width 0.4) (layer F.Cu) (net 2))
 (segment (start 162 125.6) (end 159.75 127.85) (width 0.4) (layer F.Cu) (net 2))
 (segment (start 162.05 103.8) (end 162.05 109.45) (width 0.4) (layer F.Cu) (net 2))
 (segment (start 162.05 109.45) (end 166.5 113.9) (width 0.4) (layer F.Cu) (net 2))
 (segment (start 163.698 118.286) (end 165.214 118.286) (width 0.4) (layer F.Cu) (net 2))
 (segment (start 166.5 117) (end 166.5 113.9) (width 0.4) (layer F.Cu) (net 2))
 (segment (start 165.214 118.286) (end 166.5 117) (width 0.4) (layer F.Cu) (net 2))
 (segment (start 163.698 118.286) (end 162 118.286) (width 0.4) (layer F.Cu) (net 2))
 (segment (start 162 118.286) (end 160.19 118.286) (width 0.4) (layer F.Cu) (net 2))
 (segment (start 160.19 118.286) (end 160 118.476) (width 0.4) (layer F.Cu) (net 2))
 (segment (start 160.19 118.286) (end 160 118.476) (width 1) (layer F.Cu) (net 2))
 (segment (start 149.445 113.3) (end 151.45 113.3) (width 0.4) (layer F.Cu) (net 10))
 (segment (start 151.45 113.3) (end 151.5 113.25) (width 0.4) (layer F.Cu) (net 10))
 (segment (start 146.905 113.3) (end 146.905 113.905) (width 0.4) (layer F.Cu) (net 11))
 (segment (start 146.905 113.905) (end 147.75 114.75) (width 0.4) (layer F.Cu) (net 11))
 (segment (start 147.75 114.75) (end 151.5 114.75) (width 0.4) (layer F.Cu) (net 11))
 (segment (start 148.175 113.3) (end 148.175 111.425) (width 0.4) (layer F.Cu) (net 12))
 (segment (start 148.175 111.425) (end 147.75 111) (width 0.4) (layer F.Cu) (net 12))
 (segment (start 145.635 113.3) (end 145.635 111.115) (width 0.4) (layer F.Cu) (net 13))
 (segment (start 145.635 111.115) (end 145.75 111) (width 0.4) (layer F.Cu) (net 13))
 (segment (start 145.865 111.115) (end 145.75 111) (width 0.4) (layer F.Cu) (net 13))
 (segment (start 144.365 113.3) (end 144.365 111.115) (width 0.4) (layer F.Cu) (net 14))
 (segment (start 144.365 111.115) (end 144.25 111) (width 0.4) (layer F.Cu) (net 14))
 (segment (start 143.095 113.3) (end 143.095 111.845) (width 0.4) (layer F.Cu) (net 15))
 (segment (start 143.095 111.845) (end 142.25 111) (width 0.4) (layer F.Cu) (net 15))
 (segment (start 143.095 118.7) (end 143.095 119.655) (width 0.4) (layer F.Cu) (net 8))
 (segment (start 140 120) (end 137.27 117.27) (width 0.4) (layer F.Cu) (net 8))
 (segment (start 142.75 120) (end 140 120) (width 0.4) (layer F.Cu) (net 8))
 (segment (start 143.095 119.655) (end 142.75 120) (width 0.4) (layer F.Cu) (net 8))
 (segment (start 137.27 117.27) (end 137 117.27) (width 0.4) (layer F.Cu) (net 8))
 (segment (start 144.365 118.7) (end 144.365 119.635) (width 0.4) (layer F.Cu) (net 9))
 (segment (start 137.94 120.75) (end 137 119.81) (width 0.4) (layer F.Cu) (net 9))
 (segment (start 143.25 120.75) (end 137.94 120.75) (width 0.4) (layer F.Cu) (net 9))
 (segment (start 144.365 119.635) (end 143.25 120.75) (width 0.4) (layer F.Cu) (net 9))
 (segment (start 137.19 120) (end 137 119.81) (width 0.4) (layer F.Cu) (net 9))
 (segment (start 137.19 120) (end 137 119.81) (width 0.4) (layer F.Cu) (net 9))
 (segment (start 152 126) (end 146.905 120.905) (width 0.4) (layer F.Cu) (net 7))
 (segment (start 146.905 120.905) (end 146.905 118.7) (width 0.4) (layer F.Cu) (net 7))
 (segment (start 155.5 126) (end 155.5 126.25) (width 0.4) (layer F.Cu) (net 1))
 (segment (start 155.5 126.25) (end 157.75 128.5) (width 0.4) (layer F.Cu) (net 1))
 (segment (start 157.75 128.5) (end 160.25 128.5) (width 0.4) (layer F.Cu) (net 1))
 (segment (start 160.25 128.5) (end 168.4 120.35) (width 0.4) (layer F.Cu) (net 1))
 (segment (start 168.4 120.35) (end 168.4 103.8) (width 0.4) (layer F.Cu) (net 1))
 (segment (start 148.5 126) (end 145.635 123.135) (width 0.4) (layer F.Cu) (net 6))
 (segment (start 145.635 123.135) (end 145.635 118.7) (width 0.4) (layer F.Cu) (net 6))
 (segment (start 149.445 118.7) (end 153.45 118.7) (width 0.4) (layer F.Cu) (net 5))
 (segment (start 153.45 118.7) (end 153.75 119) (width 0.4) (layer F.Cu) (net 5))
 (segment (start 153.4 116.95) (end 153.4 118.65) (width 0.4) (layer F.Cu) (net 5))
 (segment (start 153.4 118.65) (end 153.75 119) (width 0.4) (layer F.Cu) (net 5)))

